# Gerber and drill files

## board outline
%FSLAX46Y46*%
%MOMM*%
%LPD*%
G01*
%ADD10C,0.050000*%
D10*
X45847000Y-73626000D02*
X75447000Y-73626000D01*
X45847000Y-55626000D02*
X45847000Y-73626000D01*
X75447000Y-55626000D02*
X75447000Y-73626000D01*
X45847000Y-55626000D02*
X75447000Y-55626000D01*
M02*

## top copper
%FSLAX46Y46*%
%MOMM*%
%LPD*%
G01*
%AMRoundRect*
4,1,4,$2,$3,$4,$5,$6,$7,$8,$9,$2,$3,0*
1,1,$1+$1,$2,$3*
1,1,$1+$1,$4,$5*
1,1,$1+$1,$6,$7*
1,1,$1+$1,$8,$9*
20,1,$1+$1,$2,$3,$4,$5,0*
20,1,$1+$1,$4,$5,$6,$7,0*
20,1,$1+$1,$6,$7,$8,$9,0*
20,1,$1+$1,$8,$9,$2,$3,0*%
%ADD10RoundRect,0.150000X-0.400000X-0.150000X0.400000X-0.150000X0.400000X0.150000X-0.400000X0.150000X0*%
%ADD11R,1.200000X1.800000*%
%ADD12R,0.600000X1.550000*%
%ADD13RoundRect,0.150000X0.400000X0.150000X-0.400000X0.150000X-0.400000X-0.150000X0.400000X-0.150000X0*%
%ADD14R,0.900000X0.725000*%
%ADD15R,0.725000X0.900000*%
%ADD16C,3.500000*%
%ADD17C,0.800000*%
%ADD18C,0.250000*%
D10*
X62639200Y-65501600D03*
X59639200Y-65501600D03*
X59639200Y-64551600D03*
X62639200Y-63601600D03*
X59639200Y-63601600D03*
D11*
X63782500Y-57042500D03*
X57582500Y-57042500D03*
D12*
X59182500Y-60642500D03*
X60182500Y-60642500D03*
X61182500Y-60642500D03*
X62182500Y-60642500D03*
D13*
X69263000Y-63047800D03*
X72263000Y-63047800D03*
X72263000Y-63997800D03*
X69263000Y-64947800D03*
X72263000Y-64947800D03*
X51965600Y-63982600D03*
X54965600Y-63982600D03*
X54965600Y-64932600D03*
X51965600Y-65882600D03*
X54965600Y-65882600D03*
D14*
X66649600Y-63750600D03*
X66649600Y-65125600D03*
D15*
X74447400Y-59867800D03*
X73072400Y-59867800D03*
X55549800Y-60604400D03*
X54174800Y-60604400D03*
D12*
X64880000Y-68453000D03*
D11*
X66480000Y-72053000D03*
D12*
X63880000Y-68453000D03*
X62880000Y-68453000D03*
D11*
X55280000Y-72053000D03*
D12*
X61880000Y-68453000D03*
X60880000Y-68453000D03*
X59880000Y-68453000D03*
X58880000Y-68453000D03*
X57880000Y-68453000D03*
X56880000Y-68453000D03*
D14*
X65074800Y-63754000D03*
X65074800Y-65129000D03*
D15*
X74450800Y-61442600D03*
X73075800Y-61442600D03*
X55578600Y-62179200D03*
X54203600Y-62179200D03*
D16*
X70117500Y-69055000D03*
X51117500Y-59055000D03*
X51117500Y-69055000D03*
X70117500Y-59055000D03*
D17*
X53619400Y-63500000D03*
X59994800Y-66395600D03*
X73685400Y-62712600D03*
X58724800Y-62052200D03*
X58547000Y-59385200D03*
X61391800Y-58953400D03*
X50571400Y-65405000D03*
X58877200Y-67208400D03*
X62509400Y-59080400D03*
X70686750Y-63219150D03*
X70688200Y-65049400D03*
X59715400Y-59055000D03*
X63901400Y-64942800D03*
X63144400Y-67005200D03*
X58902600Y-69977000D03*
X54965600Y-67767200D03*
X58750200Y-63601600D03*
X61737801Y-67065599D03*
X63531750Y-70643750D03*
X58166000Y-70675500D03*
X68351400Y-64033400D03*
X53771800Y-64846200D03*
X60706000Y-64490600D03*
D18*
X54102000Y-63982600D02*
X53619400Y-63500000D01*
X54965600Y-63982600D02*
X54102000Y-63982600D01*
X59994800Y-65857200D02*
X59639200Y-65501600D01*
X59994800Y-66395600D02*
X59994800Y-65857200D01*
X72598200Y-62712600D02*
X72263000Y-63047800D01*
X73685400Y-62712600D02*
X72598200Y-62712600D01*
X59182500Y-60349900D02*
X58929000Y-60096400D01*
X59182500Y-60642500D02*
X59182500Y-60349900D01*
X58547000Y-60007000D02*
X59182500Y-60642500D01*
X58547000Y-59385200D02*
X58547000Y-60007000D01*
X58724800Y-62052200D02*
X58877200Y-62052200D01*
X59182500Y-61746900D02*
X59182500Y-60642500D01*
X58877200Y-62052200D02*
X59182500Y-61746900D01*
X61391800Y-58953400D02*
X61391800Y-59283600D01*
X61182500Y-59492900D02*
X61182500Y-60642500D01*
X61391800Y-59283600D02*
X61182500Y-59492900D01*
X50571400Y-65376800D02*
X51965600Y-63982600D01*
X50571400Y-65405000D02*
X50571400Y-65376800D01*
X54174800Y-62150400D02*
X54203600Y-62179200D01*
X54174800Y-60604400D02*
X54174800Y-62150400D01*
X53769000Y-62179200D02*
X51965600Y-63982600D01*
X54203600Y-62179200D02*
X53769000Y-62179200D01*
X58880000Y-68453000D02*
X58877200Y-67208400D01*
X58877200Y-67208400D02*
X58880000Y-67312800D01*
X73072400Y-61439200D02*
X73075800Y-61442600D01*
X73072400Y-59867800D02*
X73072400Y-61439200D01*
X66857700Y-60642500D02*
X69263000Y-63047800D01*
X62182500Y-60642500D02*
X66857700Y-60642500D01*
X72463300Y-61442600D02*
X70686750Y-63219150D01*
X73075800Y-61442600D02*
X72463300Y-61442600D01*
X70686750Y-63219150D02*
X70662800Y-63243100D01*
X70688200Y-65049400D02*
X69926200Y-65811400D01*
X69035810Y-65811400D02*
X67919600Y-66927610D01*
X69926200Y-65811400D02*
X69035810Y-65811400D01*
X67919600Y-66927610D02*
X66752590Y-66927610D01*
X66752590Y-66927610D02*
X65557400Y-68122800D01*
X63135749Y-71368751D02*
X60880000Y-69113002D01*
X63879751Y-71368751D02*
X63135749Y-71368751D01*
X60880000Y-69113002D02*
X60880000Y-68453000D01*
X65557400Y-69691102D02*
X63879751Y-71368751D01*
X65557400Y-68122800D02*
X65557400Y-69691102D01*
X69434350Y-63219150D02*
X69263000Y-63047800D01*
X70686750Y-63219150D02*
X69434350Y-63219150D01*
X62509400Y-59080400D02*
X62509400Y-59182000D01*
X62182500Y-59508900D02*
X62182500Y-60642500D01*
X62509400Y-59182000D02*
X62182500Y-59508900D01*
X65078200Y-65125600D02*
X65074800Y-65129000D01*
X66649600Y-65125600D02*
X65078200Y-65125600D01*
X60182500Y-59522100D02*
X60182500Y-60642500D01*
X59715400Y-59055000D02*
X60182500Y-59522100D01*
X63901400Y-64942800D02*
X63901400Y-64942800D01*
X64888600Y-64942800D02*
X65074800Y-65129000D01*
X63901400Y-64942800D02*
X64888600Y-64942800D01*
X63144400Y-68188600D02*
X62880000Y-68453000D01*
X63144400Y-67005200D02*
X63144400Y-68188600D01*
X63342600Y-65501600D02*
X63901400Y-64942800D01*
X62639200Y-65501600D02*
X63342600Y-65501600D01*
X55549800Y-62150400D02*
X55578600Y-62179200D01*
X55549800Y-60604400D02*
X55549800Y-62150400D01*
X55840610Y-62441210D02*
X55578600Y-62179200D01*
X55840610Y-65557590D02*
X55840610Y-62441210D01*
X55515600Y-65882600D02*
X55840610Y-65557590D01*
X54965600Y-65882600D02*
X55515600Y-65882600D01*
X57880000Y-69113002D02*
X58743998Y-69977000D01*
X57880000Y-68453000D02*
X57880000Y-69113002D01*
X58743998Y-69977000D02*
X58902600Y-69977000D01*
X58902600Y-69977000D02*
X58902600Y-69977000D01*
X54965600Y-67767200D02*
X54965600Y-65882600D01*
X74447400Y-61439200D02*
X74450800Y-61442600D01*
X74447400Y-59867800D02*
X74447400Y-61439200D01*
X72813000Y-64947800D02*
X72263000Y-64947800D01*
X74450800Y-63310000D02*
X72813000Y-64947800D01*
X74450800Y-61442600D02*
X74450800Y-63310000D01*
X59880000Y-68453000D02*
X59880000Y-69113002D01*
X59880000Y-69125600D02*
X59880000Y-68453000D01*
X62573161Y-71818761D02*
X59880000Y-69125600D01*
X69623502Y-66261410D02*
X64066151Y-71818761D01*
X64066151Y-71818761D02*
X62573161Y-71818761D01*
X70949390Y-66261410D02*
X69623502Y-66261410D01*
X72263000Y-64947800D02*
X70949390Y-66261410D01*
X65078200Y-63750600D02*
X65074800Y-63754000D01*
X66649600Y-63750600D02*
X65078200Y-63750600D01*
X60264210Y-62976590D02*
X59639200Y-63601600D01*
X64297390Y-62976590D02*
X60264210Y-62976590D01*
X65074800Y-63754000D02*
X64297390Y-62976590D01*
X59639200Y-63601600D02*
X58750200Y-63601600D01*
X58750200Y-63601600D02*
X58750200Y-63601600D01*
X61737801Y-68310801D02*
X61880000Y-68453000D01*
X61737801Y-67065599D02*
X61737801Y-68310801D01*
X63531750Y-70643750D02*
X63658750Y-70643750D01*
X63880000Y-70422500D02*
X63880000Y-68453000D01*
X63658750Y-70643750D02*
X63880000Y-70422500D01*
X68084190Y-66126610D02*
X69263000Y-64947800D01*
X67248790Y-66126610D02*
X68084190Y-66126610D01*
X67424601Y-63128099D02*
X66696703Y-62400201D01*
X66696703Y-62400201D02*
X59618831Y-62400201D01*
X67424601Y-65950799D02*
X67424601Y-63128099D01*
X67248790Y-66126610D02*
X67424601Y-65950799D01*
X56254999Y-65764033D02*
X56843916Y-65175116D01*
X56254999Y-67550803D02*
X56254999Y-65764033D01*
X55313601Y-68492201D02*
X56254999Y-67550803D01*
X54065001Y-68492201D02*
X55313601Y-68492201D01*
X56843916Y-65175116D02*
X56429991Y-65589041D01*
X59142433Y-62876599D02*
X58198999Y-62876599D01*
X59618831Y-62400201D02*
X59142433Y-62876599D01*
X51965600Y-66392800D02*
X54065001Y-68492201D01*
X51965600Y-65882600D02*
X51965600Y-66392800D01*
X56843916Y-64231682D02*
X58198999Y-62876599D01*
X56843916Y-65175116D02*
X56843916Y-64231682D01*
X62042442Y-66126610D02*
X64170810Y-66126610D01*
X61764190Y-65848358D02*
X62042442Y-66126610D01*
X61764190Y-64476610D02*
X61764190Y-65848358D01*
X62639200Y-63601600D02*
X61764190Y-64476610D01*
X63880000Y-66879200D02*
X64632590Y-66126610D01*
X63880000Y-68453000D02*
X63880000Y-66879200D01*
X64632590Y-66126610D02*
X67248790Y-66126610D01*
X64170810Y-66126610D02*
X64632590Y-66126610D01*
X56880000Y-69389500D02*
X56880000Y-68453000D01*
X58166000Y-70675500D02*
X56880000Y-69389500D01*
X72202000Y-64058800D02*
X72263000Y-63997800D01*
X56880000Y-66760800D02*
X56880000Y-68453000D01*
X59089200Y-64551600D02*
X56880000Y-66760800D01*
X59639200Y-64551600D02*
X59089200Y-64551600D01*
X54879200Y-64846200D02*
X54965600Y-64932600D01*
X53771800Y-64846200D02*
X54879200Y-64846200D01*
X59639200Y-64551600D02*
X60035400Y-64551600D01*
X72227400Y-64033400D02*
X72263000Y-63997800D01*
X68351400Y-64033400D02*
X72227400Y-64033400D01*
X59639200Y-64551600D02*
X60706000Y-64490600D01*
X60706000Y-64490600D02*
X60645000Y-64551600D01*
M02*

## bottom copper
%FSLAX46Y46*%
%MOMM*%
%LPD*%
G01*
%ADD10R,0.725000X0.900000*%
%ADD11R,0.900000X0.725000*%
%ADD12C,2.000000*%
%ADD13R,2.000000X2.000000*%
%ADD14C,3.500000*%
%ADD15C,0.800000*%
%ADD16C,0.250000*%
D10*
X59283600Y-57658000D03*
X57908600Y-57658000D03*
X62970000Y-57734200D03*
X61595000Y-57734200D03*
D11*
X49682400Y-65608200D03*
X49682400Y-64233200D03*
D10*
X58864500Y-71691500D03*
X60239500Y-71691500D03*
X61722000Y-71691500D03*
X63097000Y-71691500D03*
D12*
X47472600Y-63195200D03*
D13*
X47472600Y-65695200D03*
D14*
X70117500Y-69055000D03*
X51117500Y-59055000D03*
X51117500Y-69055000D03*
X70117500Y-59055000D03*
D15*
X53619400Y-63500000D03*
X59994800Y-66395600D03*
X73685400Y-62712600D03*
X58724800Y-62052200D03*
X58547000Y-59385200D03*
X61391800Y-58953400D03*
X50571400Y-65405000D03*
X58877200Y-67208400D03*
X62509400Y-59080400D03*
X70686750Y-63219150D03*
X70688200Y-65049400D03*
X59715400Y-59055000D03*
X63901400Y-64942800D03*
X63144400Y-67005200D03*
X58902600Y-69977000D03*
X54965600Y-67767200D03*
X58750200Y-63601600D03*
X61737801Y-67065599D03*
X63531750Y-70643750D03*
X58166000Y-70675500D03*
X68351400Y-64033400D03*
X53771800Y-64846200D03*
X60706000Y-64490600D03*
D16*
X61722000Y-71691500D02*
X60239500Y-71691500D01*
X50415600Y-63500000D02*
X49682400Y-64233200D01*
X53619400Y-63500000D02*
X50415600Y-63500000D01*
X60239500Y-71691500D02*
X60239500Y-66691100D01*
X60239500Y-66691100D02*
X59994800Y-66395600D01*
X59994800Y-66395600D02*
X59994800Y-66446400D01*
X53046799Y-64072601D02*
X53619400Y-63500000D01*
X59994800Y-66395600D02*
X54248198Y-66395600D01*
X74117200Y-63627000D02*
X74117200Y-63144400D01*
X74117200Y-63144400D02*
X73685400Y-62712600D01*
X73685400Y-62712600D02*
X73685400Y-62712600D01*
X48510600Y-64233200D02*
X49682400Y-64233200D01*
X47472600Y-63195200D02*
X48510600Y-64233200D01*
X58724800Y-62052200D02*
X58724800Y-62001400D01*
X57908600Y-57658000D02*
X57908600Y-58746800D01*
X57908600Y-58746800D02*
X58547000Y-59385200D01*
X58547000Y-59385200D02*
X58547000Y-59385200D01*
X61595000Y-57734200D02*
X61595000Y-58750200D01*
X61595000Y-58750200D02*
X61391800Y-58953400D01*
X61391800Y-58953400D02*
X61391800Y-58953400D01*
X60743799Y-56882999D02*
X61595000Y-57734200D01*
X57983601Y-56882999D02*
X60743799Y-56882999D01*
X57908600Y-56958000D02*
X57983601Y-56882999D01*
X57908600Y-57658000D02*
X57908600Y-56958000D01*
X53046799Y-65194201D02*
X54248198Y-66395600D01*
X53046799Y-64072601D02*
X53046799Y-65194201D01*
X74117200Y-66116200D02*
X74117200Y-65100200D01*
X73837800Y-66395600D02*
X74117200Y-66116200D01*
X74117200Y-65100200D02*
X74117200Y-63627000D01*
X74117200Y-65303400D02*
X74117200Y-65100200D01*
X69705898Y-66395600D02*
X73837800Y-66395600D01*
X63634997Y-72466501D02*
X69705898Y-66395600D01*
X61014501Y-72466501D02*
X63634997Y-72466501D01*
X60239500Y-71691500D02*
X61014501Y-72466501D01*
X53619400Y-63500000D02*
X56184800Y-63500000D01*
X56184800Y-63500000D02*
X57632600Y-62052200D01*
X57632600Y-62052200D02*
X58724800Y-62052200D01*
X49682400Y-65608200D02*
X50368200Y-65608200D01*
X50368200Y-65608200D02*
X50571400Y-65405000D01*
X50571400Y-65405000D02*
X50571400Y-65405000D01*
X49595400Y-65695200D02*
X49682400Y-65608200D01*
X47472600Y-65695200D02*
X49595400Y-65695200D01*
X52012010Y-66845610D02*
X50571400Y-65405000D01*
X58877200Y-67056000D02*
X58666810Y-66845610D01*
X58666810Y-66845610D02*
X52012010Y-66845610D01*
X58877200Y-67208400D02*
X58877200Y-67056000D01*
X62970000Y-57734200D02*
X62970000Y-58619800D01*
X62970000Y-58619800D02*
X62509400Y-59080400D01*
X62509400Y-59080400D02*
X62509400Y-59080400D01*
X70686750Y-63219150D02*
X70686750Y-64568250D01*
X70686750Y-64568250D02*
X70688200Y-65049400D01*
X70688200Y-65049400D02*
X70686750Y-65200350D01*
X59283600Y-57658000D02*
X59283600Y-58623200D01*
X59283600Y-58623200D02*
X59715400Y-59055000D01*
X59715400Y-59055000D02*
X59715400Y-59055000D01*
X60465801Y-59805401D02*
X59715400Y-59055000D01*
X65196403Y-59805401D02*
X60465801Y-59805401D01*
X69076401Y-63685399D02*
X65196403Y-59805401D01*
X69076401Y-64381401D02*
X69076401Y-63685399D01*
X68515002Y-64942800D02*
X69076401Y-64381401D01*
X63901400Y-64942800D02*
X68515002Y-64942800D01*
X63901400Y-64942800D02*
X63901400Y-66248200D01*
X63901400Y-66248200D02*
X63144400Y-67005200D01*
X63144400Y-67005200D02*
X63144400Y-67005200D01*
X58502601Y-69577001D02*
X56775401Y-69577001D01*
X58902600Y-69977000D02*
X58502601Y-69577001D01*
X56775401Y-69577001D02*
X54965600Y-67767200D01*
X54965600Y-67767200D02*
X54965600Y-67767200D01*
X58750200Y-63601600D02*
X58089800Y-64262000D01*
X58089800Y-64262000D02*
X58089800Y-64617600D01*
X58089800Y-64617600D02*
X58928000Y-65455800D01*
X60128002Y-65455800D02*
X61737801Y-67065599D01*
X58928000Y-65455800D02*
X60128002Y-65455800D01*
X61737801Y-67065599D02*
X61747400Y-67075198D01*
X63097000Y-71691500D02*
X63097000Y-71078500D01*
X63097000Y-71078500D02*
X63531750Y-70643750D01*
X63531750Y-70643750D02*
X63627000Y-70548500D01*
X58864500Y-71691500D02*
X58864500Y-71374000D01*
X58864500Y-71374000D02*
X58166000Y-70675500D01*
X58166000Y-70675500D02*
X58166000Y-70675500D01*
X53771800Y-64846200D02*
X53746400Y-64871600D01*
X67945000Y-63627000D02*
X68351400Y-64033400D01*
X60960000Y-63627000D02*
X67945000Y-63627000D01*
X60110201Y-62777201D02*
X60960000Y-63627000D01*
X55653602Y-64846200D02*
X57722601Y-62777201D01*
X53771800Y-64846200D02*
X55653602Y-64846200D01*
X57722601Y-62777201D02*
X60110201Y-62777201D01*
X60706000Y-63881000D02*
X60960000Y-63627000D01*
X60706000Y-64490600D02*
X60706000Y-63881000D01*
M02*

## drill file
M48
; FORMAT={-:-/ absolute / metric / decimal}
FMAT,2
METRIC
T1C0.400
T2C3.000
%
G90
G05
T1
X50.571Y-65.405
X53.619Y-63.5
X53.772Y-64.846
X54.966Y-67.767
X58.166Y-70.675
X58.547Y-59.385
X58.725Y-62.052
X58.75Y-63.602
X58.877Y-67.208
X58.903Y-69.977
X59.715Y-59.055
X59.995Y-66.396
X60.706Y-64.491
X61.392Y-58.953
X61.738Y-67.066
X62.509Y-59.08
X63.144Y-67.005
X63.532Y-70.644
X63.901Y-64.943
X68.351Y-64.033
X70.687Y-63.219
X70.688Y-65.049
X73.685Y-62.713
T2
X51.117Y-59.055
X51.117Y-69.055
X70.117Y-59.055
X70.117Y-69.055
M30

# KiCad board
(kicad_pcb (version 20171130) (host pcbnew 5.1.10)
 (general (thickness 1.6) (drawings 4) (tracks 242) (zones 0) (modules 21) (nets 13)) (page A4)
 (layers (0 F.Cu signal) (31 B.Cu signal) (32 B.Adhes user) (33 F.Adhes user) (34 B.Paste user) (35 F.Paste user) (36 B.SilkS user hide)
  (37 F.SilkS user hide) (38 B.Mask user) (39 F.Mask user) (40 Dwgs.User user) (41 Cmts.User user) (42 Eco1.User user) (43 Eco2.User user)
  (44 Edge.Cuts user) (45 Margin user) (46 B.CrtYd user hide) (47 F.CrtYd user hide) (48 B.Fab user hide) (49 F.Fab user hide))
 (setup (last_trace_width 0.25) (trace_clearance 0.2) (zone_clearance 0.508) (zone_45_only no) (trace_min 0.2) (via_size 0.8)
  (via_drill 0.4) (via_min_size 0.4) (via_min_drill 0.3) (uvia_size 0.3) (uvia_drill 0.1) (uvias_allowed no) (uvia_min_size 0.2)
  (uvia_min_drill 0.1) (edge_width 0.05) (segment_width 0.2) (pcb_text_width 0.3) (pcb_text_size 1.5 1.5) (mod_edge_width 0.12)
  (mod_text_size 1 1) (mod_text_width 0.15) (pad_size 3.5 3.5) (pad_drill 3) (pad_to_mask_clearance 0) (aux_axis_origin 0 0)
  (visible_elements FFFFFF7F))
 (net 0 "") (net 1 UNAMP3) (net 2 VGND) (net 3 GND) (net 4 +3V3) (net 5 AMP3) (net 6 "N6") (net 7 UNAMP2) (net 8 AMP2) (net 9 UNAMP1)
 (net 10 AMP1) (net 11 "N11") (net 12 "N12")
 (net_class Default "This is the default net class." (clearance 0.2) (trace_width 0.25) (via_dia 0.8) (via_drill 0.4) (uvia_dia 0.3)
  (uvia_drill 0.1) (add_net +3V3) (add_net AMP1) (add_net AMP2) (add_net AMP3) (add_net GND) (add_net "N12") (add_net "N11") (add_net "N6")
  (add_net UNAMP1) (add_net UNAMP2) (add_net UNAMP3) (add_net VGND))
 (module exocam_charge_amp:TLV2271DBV (layer F.Cu) (at 60.9092 61.0616)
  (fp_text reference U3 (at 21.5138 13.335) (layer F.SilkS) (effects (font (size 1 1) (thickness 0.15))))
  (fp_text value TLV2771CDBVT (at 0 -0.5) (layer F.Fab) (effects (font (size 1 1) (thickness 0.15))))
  (pad 4 smd roundrect (at 1.73 4.44) (size 1.1 0.6) (layers F.Cu F.Paste F.Mask) (roundrect_rratio 0.25) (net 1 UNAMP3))
  (pad 3 smd roundrect (at -1.27 4.44) (size 1.1 0.6) (layers F.Cu F.Paste F.Mask) (roundrect_rratio 0.25) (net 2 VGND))
  (pad 2 smd roundrect (at -1.27 3.49) (size 1.1 0.6) (layers F.Cu F.Paste F.Mask) (roundrect_rratio 0.25) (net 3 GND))
  (pad 5 smd roundrect (at 1.73 2.54) (size 1.1 0.6) (layers F.Cu F.Paste F.Mask) (roundrect_rratio 0.25) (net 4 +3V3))
  (pad 1 smd roundrect (at -1.27 2.54) (size 1.1 0.6) (layers F.Cu F.Paste F.Mask) (roundrect_rratio 0.25) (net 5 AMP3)))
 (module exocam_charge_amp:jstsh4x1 (layer F.Cu) (at 59.3725 63.1825 180)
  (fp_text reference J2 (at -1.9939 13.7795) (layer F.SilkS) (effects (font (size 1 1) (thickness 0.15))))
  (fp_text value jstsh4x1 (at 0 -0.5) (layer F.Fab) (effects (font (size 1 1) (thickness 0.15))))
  (pad 5 smd rect (at -4.41 6.14 180) (size 1.2 1.8) (layers F.Cu F.Paste F.Mask) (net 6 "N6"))
  (pad 5 smd rect (at 1.79 6.14 180) (size 1.2 1.8) (layers F.Cu F.Paste F.Mask) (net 6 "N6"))
  (pad 4 smd rect (at 0.19 2.54 180) (size 0.6 1.55) (layers F.Cu F.Paste F.Mask) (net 2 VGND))
  (pad 3 smd rect (at -0.81 2.54 180) (size 0.6 1.55) (layers F.Cu F.Paste F.Mask) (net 1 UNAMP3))
  (pad 2 smd rect (at -1.81 2.54 180) (size 0.6 1.55) (layers F.Cu F.Paste F.Mask) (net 2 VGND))
  (pad 1 smd rect (at -2.81 2.54 180) (size 0.6 1.55) (layers F.Cu F.Paste F.Mask) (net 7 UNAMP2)))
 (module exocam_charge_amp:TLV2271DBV (layer F.Cu) (at 70.993 67.4878 180)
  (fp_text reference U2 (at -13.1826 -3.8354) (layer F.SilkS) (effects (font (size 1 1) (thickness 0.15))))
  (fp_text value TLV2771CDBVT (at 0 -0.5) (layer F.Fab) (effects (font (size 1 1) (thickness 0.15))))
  (pad 4 smd roundrect (at 1.73 4.44 180) (size 1.1 0.6) (layers F.Cu F.Paste F.Mask) (roundrect_rratio 0.25) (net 7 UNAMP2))
  (pad 3 smd roundrect (at -1.27 4.44 180) (size 1.1 0.6) (layers F.Cu F.Paste F.Mask) (roundrect_rratio 0.25) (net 2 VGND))
  (pad 2 smd roundrect (at -1.27 3.49 180) (size 1.1 0.6) (layers F.Cu F.Paste F.Mask) (roundrect_rratio 0.25) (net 3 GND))
  (pad 5 smd roundrect (at 1.73 2.54 180) (size 1.1 0.6) (layers F.Cu F.Paste F.Mask) (roundrect_rratio 0.25) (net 4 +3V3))
  (pad 1 smd roundrect (at -1.27 2.54 180) (size 1.1 0.6) (layers F.Cu F.Paste F.Mask) (roundrect_rratio 0.25) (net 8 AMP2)))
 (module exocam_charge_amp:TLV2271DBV (layer F.Cu) (at 53.6956 68.4226 180)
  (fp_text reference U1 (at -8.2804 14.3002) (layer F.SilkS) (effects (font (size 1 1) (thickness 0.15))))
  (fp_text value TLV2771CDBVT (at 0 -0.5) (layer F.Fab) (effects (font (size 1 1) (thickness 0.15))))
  (pad 4 smd roundrect (at 1.73 4.44 180) (size 1.1 0.6) (layers F.Cu F.Paste F.Mask) (roundrect_rratio 0.25) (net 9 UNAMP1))
  (pad 3 smd roundrect (at -1.27 4.44 180) (size 1.1 0.6) (layers F.Cu F.Paste F.Mask) (roundrect_rratio 0.25) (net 2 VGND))
  (pad 2 smd roundrect (at -1.27 3.49 180) (size 1.1 0.6) (layers F.Cu F.Paste F.Mask) (roundrect_rratio 0.25) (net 3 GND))
  (pad 5 smd roundrect (at 1.73 2.54 180) (size 1.1 0.6) (layers F.Cu F.Paste F.Mask) (roundrect_rratio 0.25) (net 4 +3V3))
  (pad 1 smd roundrect (at -1.27 2.54 180) (size 1.1 0.6) (layers F.Cu F.Paste F.Mask) (roundrect_rratio 0.25) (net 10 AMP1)))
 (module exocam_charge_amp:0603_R (layer F.Cu) (at 64.1096 63.8556 90)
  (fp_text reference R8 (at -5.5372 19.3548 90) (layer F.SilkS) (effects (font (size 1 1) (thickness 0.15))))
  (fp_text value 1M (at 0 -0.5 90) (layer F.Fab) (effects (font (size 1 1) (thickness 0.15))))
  (pad 2 smd rect (at 0.105 2.54 90) (size 0.725 0.9) (layers F.Cu F.Paste F.Mask) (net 5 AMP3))
  (pad 1 smd rect (at -1.27 2.54 90) (size 0.725 0.9) (layers F.Cu F.Paste F.Mask) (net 1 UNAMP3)))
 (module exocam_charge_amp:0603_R (layer B.Cu) (at 59.1786 60.198)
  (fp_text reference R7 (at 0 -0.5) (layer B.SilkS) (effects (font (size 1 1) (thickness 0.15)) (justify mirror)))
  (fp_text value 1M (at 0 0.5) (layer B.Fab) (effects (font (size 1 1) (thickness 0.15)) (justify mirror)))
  (pad 2 smd rect (at 0.105 -2.54) (size 0.725 0.9) (layers B.Cu B.Paste B.Mask) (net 1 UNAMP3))
  (pad 1 smd rect (at -1.27 -2.54) (size 0.725 0.9) (layers B.Cu B.Paste B.Mask) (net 2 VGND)))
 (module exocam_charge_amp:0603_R (layer F.Cu) (at 74.3424 57.3278)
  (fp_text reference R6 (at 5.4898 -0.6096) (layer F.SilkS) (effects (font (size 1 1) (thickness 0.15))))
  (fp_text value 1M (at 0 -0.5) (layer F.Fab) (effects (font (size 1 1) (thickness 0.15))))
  (pad 2 smd rect (at 0.105 2.54) (size 0.725 0.9) (layers F.Cu F.Paste F.Mask) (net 8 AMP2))
  (pad 1 smd rect (at -1.27 2.54) (size 0.725 0.9) (layers F.Cu F.Paste F.Mask) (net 7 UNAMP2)))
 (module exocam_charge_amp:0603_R (layer B.Cu) (at 62.865 60.2742)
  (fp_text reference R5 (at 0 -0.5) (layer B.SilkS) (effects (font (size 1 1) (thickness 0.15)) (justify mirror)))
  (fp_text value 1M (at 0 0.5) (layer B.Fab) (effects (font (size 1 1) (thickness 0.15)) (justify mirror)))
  (pad 2 smd rect (at 0.105 -2.54) (size 0.725 0.9) (layers B.Cu B.Paste B.Mask) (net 7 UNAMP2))
  (pad 1 smd rect (at -1.27 -2.54) (size 0.725 0.9) (layers B.Cu B.Paste B.Mask) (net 2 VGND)))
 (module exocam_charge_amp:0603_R (layer B.Cu) (at 47.1424 65.5032 270)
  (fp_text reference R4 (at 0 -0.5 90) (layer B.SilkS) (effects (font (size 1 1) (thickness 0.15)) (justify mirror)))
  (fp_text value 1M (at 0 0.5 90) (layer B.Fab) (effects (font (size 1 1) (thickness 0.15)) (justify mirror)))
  (pad 2 smd rect (at 0.105 -2.54 270) (size 0.725 0.9) (layers B.Cu B.Paste B.Mask) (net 9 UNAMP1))
  (pad 1 smd rect (at -1.27 -2.54 270) (size 0.725 0.9) (layers B.Cu B.Paste B.Mask) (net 2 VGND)))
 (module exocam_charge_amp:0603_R (layer F.Cu) (at 55.4448 58.0644)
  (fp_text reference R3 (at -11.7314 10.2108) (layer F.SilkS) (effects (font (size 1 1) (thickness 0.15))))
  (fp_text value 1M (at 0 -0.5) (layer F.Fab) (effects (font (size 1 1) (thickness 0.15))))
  (pad 2 smd rect (at 0.105 2.54) (size 0.725 0.9) (layers F.Cu F.Paste F.Mask) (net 10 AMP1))
  (pad 1 smd rect (at -1.27 2.54) (size 0.725 0.9) (layers F.Cu F.Paste F.Mask) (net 9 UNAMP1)))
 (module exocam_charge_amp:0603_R (layer B.Cu) (at 58.9695 69.1515 180)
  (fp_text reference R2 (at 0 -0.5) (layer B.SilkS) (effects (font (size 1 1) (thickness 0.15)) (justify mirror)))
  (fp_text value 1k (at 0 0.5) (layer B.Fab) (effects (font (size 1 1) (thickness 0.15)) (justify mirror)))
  (pad 2 smd rect (at 0.105 -2.54 180) (size 0.725 0.9) (layers B.Cu B.Paste B.Mask) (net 3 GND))
  (pad 1 smd rect (at -1.27 -2.54 180) (size 0.725 0.9) (layers B.Cu B.Paste B.Mask) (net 2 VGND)))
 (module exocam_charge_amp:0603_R (layer B.Cu) (at 61.827 69.1515 180)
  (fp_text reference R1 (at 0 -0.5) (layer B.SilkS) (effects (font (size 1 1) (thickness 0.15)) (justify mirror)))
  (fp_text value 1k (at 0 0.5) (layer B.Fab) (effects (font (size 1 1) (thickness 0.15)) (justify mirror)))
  (pad 2 smd rect (at 0.105 -2.54 180) (size 0.725 0.9) (layers B.Cu B.Paste B.Mask) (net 2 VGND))
  (pad 1 smd rect (at -1.27 -2.54 180) (size 0.725 0.9) (layers B.Cu B.Paste B.Mask) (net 4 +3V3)))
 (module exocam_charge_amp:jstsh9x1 (layer F.Cu) (at 59.69 65.913)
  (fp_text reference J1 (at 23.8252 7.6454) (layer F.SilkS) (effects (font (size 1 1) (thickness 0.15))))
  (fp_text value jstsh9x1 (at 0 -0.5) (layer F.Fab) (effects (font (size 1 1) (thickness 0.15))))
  (pad 9 smd rect (at 5.19 2.54) (size 0.6 1.55) (layers F.Cu F.Paste F.Mask) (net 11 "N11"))
  (pad 10 smd rect (at 6.79 6.14) (size 1.2 1.8) (layers F.Cu F.Paste F.Mask) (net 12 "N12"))
  (pad 8 smd rect (at 4.19 2.54) (size 0.6 1.55) (layers F.Cu F.Paste F.Mask) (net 4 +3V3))
  (pad 7 smd rect (at 3.19 2.54) (size 0.6 1.55) (layers F.Cu F.Paste F.Mask) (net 1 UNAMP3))
  (pad 10 smd rect (at -4.41 6.14) (size 1.2 1.8) (layers F.Cu F.Paste F.Mask) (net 12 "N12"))
  (pad 6 smd rect (at 2.19 2.54) (size 0.6 1.55) (layers F.Cu F.Paste F.Mask) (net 5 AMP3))
  (pad 5 smd rect (at 1.19 2.54) (size 0.6 1.55) (layers F.Cu F.Paste F.Mask) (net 7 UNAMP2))
  (pad 4 smd rect (at 0.19 2.54) (size 0.6 1.55) (layers F.Cu F.Paste F.Mask) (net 8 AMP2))
  (pad 3 smd rect (at -0.81 2.54) (size 0.6 1.55) (layers F.Cu F.Paste F.Mask) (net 9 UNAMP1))
  (pad 2 smd rect (at -1.81 2.54) (size 0.6 1.55) (layers F.Cu F.Paste F.Mask) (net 10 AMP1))
  (pad 1 smd rect (at -2.81 2.54) (size 0.6 1.55) (layers F.Cu F.Paste F.Mask) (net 3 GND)))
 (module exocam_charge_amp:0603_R (layer F.Cu) (at 62.5348 63.859 90)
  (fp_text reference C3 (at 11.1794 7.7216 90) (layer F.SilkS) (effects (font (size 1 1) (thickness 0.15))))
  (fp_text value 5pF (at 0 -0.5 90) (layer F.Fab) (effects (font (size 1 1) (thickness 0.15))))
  (pad 2 smd rect (at 0.105 2.54 90) (size 0.725 0.9) (layers F.Cu F.Paste F.Mask) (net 5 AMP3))
  (pad 1 smd rect (at -1.27 2.54 90) (size 0.725 0.9) (layers F.Cu F.Paste F.Mask) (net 1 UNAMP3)))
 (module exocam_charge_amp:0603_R (layer F.Cu) (at 74.3458 58.9026)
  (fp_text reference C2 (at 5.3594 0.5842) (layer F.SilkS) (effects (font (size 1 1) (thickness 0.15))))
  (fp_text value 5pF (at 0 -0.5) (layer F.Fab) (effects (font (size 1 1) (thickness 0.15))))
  (pad 2 smd rect (at 0.105 2.54) (size 0.725 0.9) (layers F.Cu F.Paste F.Mask) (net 8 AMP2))
  (pad 1 smd rect (at -1.27 2.54) (size 0.725 0.9) (layers F.Cu F.Paste F.Mask) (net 7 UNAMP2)))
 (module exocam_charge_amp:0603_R (layer F.Cu) (at 55.4736 59.6392)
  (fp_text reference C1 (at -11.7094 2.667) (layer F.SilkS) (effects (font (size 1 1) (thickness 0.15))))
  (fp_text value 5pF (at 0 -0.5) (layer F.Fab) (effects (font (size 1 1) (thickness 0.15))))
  (pad 2 smd rect (at 0.105 2.54) (size 0.725 0.9) (layers F.Cu F.Paste F.Mask) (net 10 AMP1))
  (pad 1 smd rect (at -1.27 2.54) (size 0.725 0.9) (layers F.Cu F.Paste F.Mask) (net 9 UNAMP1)))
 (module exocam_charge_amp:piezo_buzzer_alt (layer B.Cu) (at 50.0126 64.1552 90)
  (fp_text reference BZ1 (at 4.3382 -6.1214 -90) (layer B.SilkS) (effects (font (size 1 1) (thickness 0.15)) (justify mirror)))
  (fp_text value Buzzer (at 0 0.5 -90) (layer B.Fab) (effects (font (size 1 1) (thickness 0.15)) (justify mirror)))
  (pad 2 smd circle (at 0.96 -2.54 90) (size 2 2) (layers B.Cu B.Paste B.Mask) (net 2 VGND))
  (pad 1 smd rect (at -1.54 -2.54 90) (size 2 2) (layers B.Cu B.Paste B.Mask) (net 9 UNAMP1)))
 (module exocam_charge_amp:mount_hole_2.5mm (layer F.Cu) (at 66.1035 71.501 90)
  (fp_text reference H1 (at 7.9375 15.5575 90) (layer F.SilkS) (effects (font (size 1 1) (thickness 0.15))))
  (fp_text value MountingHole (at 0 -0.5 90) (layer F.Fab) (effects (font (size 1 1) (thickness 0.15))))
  (pad 1 thru_hole circle (at 2.446 4.014 90) (size 3.5 3.5) (drill 3) (layers *.Cu *.Mask)))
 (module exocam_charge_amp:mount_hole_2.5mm (layer F.Cu) (at 47.3075 57.785 90)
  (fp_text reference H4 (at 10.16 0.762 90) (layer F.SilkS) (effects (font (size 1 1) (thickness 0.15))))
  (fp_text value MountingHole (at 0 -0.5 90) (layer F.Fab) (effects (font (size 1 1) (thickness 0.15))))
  (pad 1 thru_hole circle (at -1.27 3.81 90) (size 3.5 3.5) (drill 3) (layers *.Cu *.Mask)))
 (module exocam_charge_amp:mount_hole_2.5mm (layer F.Cu) (at 47.3075 60.96 90)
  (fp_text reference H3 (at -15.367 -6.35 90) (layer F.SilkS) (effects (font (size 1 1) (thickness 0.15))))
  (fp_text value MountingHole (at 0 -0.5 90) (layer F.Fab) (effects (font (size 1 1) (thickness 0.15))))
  (pad 1 thru_hole circle (at -8.095 3.81 90) (size 3.5 3.5) (drill 3) (layers *.Cu *.Mask)))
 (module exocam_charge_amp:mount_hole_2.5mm (layer F.Cu) (at 66.1035 57.501 90)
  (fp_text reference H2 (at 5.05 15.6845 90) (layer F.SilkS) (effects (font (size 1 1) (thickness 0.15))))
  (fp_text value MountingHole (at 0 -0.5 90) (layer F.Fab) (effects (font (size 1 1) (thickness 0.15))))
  (pad 1 thru_hole circle (at -1.554 4.014 90) (size 3.5 3.5) (drill 3) (layers *.Cu *.Mask)))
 (gr_line (start 45.847 73.626) (end 75.447 73.626) (layer Edge.Cuts) (width 0.05))
 (gr_line (start 45.847 55.626) (end 45.847 73.626) (layer Edge.Cuts) (width 0.05))
 (gr_line (start 75.447 55.626) (end 75.447 73.626) (layer Edge.Cuts) (width 0.05))
 (gr_line (start 45.847 55.626) (end 75.447 55.626) (layer Edge.Cuts) (width 0.05))
 (segment (start 61.722 71.6915) (end 60.2395 71.6915) (width 0.25) (layer B.Cu) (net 2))
 (via (at 53.6194 63.5) (size 0.8) (drill 0.4) (layers F.Cu B.Cu) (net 2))
 (segment (start 54.102 63.9826) (end 53.6194 63.5) (width 0.25) (layer F.Cu) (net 2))
 (segment (start 54.9656 63.9826) (end 54.102 63.9826) (width 0.25) (layer F.Cu) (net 2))
 (segment (start 50.4156 63.5) (end 49.6824 64.2332) (width 0.25) (layer B.Cu) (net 2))
 (segment (start 53.6194 63.5) (end 50.4156 63.5) (width 0.25) (layer B.Cu) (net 2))
 (segment (start 60.2395 71.6915) (end 60.2395 66.6911) (width 0.25) (layer B.Cu) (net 2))
 (segment (start 60.2395 66.6911) (end 59.9948 66.3956) (width 0.25) (layer B.Cu) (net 2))
 (segment (start 59.9948 66.3956) (end 59.9948 66.4464) (width 0.25) (layer B.Cu) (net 2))
 (via (at 59.9948 66.3956) (size 0.8) (drill 0.4) (layers F.Cu B.Cu) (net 2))
 (segment (start 59.9948 65.8572) (end 59.6392 65.5016) (width 0.25) (layer F.Cu) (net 2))
 (segment (start 59.9948 66.3956) (end 59.9948 65.8572) (width 0.25) (layer F.Cu) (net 2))
 (segment (start 53.046799 64.072601) (end 53.6194 63.5) (width 0.25) (layer B.Cu) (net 2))
 (segment (start 59.9948 66.3956) (end 54.248198 66.3956) (width 0.25) (layer B.Cu) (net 2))
 (segment (start 74.1172 63.627) (end 74.1172 63.1444) (width 0.25) (layer B.Cu) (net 2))
 (segment (start 74.1172 63.1444) (end 73.6854 62.7126) (width 0.25) (layer B.Cu) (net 2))
 (segment (start 73.6854 62.7126) (end 73.6854 62.7126) (width 0.25) (layer B.Cu) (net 2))
 (via (at 73.6854 62.7126) (size 0.8) (drill 0.4) (layers F.Cu B.Cu) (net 2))
 (segment (start 72.5982 62.7126) (end 72.263 63.0478) (width 0.25) (layer F.Cu) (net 2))
 (segment (start 73.6854 62.7126) (end 72.5982 62.7126) (width 0.25) (layer F.Cu) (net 2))
 (segment (start 48.5106 64.2332) (end 49.6824 64.2332) (width 0.25) (layer B.Cu) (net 2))
 (segment (start 47.4726 63.1952) (end 48.5106 64.2332) (width 0.25) (layer B.Cu) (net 2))
 (segment (start 58.7248 62.0522) (end 58.7248 62.0014) (width 0.25) (layer B.Cu) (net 2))
 (via (at 58.7248 62.0522) (size 0.8) (drill 0.4) (layers F.Cu B.Cu) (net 2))
 (segment (start 59.1825 60.3499) (end 58.929 60.0964) (width 0.25) (layer F.Cu) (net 2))
 (segment (start 59.1825 60.6425) (end 59.1825 60.3499) (width 0.25) (layer F.Cu) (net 2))
 (segment (start 57.9086 57.658) (end 57.9086 58.7468) (width 0.25) (layer B.Cu) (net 2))
 (segment (start 57.9086 58.7468) (end 58.547 59.3852) (width 0.25) (layer B.Cu) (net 2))
 (segment (start 58.547 59.3852) (end 58.547 59.3852) (width 0.25) (layer B.Cu) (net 2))
 (via (at 58.547 59.3852) (size 0.8) (drill 0.4) (layers F.Cu B.Cu) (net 2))
 (segment (start 58.547 60.007) (end 59.1825 60.6425) (width 0.25) (layer F.Cu) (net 2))
 (segment (start 58.547 59.3852) (end 58.547 60.007) (width 0.25) (layer F.Cu) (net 2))
 (segment (start 61.595 57.7342) (end 61.595 58.7502) (width 0.25) (layer B.Cu) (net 2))
 (segment (start 61.595 58.7502) (end 61.3918 58.9534) (width 0.25) (layer B.Cu) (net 2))
 (segment (start 61.3918 58.9534) (end 61.3918 58.9534) (width 0.25) (layer B.Cu) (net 2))
 (via (at 61.3918 58.9534) (size 0.8) (drill 0.4) (layers F.Cu B.Cu) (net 2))
 (segment (start 60.743799 56.882999) (end 61.595 57.7342) (width 0.25) (layer B.Cu) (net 2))
 (segment (start 57.983601 56.882999) (end 60.743799 56.882999) (width 0.25) (layer B.Cu) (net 2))
 (segment (start 57.9086 56.958) (end 57.983601 56.882999) (width 0.25) (layer B.Cu) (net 2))
 (segment (start 57.9086 57.658) (end 57.9086 56.958) (width 0.25) (layer B.Cu) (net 2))
 (segment (start 53.046799 65.194201) (end 54.248198 66.3956) (width 0.25) (layer B.Cu) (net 2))
 (segment (start 53.046799 64.072601) (end 53.046799 65.194201) (width 0.25) (layer B.Cu) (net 2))
 (segment (start 74.1172 66.1162) (end 74.1172 65.1002) (width 0.25) (layer B.Cu) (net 2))
 (segment (start 73.8378 66.3956) (end 74.1172 66.1162) (width 0.25) (layer B.Cu) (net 2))
 (segment (start 74.1172 65.1002) (end 74.1172 63.627) (width 0.25) (layer B.Cu) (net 2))
 (segment (start 74.1172 65.3034) (end 74.1172 65.1002) (width 0.25) (layer B.Cu) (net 2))
 (segment (start 69.705898 66.3956) (end 73.8378 66.3956) (width 0.25) (layer B.Cu) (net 2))
 (segment (start 63.634997 72.466501) (end 69.705898 66.3956) (width 0.25) (layer B.Cu) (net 2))
 (segment (start 61.014501 72.466501) (end 63.634997 72.466501) (width 0.25) (layer B.Cu) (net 2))
 (segment (start 60.2395 71.6915) (end 61.014501 72.466501) (width 0.25) (layer B.Cu) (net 2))
 (segment (start 53.6194 63.5) (end 56.1848 63.5) (width 0.25) (layer B.Cu) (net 2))
 (segment (start 56.1848 63.5) (end 57.6326 62.0522) (width 0.25) (layer B.Cu) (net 2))
 (segment (start 57.6326 62.0522) (end 58.7248 62.0522) (width 0.25) (layer B.Cu) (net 2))
 (segment (start 58.7248 62.0522) (end 58.8772 62.0522) (width 0.25) (layer F.Cu) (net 2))
 (segment (start 59.1825 61.7469) (end 59.1825 60.6425) (width 0.25) (layer F.Cu) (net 2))
 (segment (start 58.8772 62.0522) (end 59.1825 61.7469) (width 0.25) (layer F.Cu) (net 2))
 (segment (start 61.3918 58.9534) (end 61.3918 59.2836) (width 0.25) (layer F.Cu) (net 2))
 (segment (start 61.1825 59.4929) (end 61.1825 60.6425) (width 0.25) (layer F.Cu) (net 2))
 (segment (start 61.3918 59.2836) (end 61.1825 59.4929) (width 0.25) (layer F.Cu) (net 2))
 (segment (start 49.6824 65.6082) (end 50.3682 65.6082) (width 0.25) (layer B.Cu) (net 9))
 (segment (start 50.3682 65.6082) (end 50.5714 65.405) (width 0.25) (layer B.Cu) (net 9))
 (segment (start 50.5714 65.405) (end 50.5714 65.405) (width 0.25) (layer B.Cu) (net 9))
 (via (at 50.5714 65.405) (size 0.8) (drill 0.4) (layers F.Cu B.Cu) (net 9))
 (segment (start 50.5714 65.3768) (end 51.9656 63.9826) (width 0.25) (layer F.Cu) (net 9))
 (segment (start 50.5714 65.405) (end 50.5714 65.3768) (width 0.25) (layer F.Cu) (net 9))
 (segment (start 54.1748 62.1504) (end 54.2036 62.1792) (width 0.25) (layer F.Cu) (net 9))
 (segment (start 54.1748 60.6044) (end 54.1748 62.1504) (width 0.25) (layer F.Cu) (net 9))
 (segment (start 53.769 62.1792) (end 51.9656 63.9826) (width 0.25) (layer F.Cu) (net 9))
 (segment (start 54.2036 62.1792) (end 53.769 62.1792) (width 0.25) (layer F.Cu) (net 9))
 (segment (start 49.5954 65.6952) (end 49.6824 65.6082) (width 0.25) (layer B.Cu) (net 9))
 (segment (start 47.4726 65.6952) (end 49.5954 65.6952) (width 0.25) (layer B.Cu) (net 9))
 (segment (start 58.88 68.453) (end 58.8772 67.2084) (width 0.25) (layer F.Cu) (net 9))
 (segment (start 58.8772 67.2084) (end 58.88 67.3128) (width 0.25) (layer F.Cu) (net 9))
 (via (at 58.8772 67.2084) (size 0.8) (drill 0.4) (layers F.Cu B.Cu) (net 9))
 (segment (start 52.01201 66.84561) (end 50.5714 65.405) (width 0.25) (layer B.Cu) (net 9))
 (segment (start 58.8772 67.056) (end 58.66681 66.84561) (width 0.25) (layer B.Cu) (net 9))
 (segment (start 58.66681 66.84561) (end 52.01201 66.84561) (width 0.25) (layer B.Cu) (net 9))
 (segment (start 58.8772 67.2084) (end 58.8772 67.056) (width 0.25) (layer B.Cu) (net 9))
 (segment (start 73.0724 61.4392) (end 73.0758 61.4426) (width 0.25) (layer F.Cu) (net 7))
 (segment (start 73.0724 59.8678) (end 73.0724 61.4392) (width 0.25) (layer F.Cu) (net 7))
 (segment (start 66.8577 60.6425) (end 69.263 63.0478) (width 0.25) (layer F.Cu) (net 7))
 (segment (start 62.1825 60.6425) (end 66.8577 60.6425) (width 0.25) (layer F.Cu) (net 7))
 (segment (start 62.97 57.7342) (end 62.97 58.6198) (width 0.25) (layer B.Cu) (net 7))
 (segment (start 62.97 58.6198) (end 62.5094 59.0804) (width 0.25) (layer B.Cu) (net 7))
 (segment (start 62.5094 59.0804) (end 62.5094 59.0804) (width 0.25) (layer B.Cu) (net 7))
 (via (at 62.5094 59.0804) (size 0.8) (drill 0.4) (layers F.Cu B.Cu) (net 7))
 (segment (start 72.4633 61.4426) (end 70.68675 63.21915) (width 0.25) (layer F.Cu) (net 7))
 (segment (start 73.0758 61.4426) (end 72.4633 61.4426) (width 0.25) (layer F.Cu) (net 7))
 (segment (start 70.68675 63.21915) (end 70.6628 63.2431) (width 0.25) (layer F.Cu) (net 7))
 (via (at 70.68675 63.21915) (size 0.8) (drill 0.4) (layers F.Cu B.Cu) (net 7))
 (segment (start 70.68675 63.21915) (end 70.68675 64.56825) (width 0.25) (layer B.Cu) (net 7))
 (segment (start 70.68675 64.56825) (end 70.6882 65.0494) (width 0.25) (layer B.Cu) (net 7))
 (segment (start 70.6882 65.0494) (end 70.68675 65.20035) (width 0.25) (layer B.Cu) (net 7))
 (via (at 70.6882 65.0494) (size 0.8) (drill 0.4) (layers F.Cu B.Cu) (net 7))
 (segment (start 70.6882 65.0494) (end 69.9262 65.8114) (width 0.25) (layer F.Cu) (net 7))
 (segment (start 69.03581 65.8114) (end 67.9196 66.92761) (width 0.25) (layer F.Cu) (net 7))
 (segment (start 69.9262 65.8114) (end 69.03581 65.8114) (width 0.25) (layer F.Cu) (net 7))
 (segment (start 67.9196 66.92761) (end 66.75259 66.92761) (width 0.25) (layer F.Cu) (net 7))
 (segment (start 66.75259 66.92761) (end 65.5574 68.1228) (width 0.25) (layer F.Cu) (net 7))
 (segment (start 63.135749 71.368751) (end 60.88 69.113002) (width 0.25) (layer F.Cu) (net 7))
 (segment (start 63.879751 71.368751) (end 63.135749 71.368751) (width 0.25) (layer F.Cu) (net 7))
 (segment (start 60.88 69.113002) (end 60.88 68.453) (width 0.25) (layer F.Cu) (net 7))
 (segment (start 65.5574 69.691102) (end 63.879751 71.368751) (width 0.25) (layer F.Cu) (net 7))
 (segment (start 65.5574 68.1228) (end 65.5574 69.691102) (width 0.25) (layer F.Cu) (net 7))
 (segment (start 69.43435 63.21915) (end 69.263 63.0478) (width 0.25) (layer F.Cu) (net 7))
 (segment (start 70.68675 63.21915) (end 69.43435 63.21915) (width 0.25) (layer F.Cu) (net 7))
 (segment (start 62.5094 59.0804) (end 62.5094 59.182) (width 0.25) (layer F.Cu) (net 7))
 (segment (start 62.1825 59.5089) (end 62.1825 60.6425) (width 0.25) (layer F.Cu) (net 7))
 (segment (start 62.5094 59.182) (end 62.1825 59.5089) (width 0.25) (layer F.Cu) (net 7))
 (segment (start 65.0782 65.1256) (end 65.0748 65.129) (width 0.25) (layer F.Cu) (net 1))
 (segment (start 66.6496 65.1256) (end 65.0782 65.1256) (width 0.25) (layer F.Cu) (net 1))
 (segment (start 59.2836 57.658) (end 59.2836 58.6232) (width 0.25) (layer B.Cu) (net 1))
 (segment (start 59.2836 58.6232) (end 59.7154 59.055) (width 0.25) (layer B.Cu) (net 1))
 (segment (start 59.7154 59.055) (end 59.7154 59.055) (width 0.25) (layer B.Cu) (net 1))
 (via (at 59.7154 59.055) (size 0.8) (drill 0.4) (layers F.Cu B.Cu) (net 1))
 (segment (start 60.1825 59.5221) (end 60.1825 60.6425) (width 0.25) (layer F.Cu) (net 1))
 (segment (start 59.7154 59.055) (end 60.1825 59.5221) (width 0.25) (layer F.Cu) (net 1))
 (segment (start 63.9014 64.9428) (end 63.9014 64.9428) (width 0.25) (layer F.Cu) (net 1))
 (via (at 63.9014 64.9428) (size 0.8) (drill 0.4) (layers F.Cu B.Cu) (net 1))
 (segment (start 60.465801 59.805401) (end 59.7154 59.055) (width 0.25) (layer B.Cu) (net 1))
 (segment (start 65.196403 59.805401) (end 60.465801 59.805401) (width 0.25) (layer B.Cu) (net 1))
 (segment (start 69.076401 63.685399) (end 65.196403 59.805401) (width 0.25) (layer B.Cu) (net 1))
 (segment (start 69.076401 64.381401) (end 69.076401 63.685399) (width 0.25) (layer B.Cu) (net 1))
 (segment (start 68.515002 64.9428) (end 69.076401 64.381401) (width 0.25) (layer B.Cu) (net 1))
 (segment (start 63.9014 64.9428) (end 68.515002 64.9428) (width 0.25) (layer B.Cu) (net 1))
 (segment (start 64.8886 64.9428) (end 65.0748 65.129) (width 0.25) (layer F.Cu) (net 1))
 (segment (start 63.9014 64.9428) (end 64.8886 64.9428) (width 0.25) (layer F.Cu) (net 1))
 (segment (start 63.9014 64.9428) (end 63.9014 66.2482) (width 0.25) (layer B.Cu) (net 1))
 (segment (start 63.9014 66.2482) (end 63.1444 67.0052) (width 0.25) (layer B.Cu) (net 1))
 (segment (start 63.1444 67.0052) (end 63.1444 67.0052) (width 0.25) (layer B.Cu) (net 1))
 (via (at 63.1444 67.0052) (size 0.8) (drill 0.4) (layers F.Cu B.Cu) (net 1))
 (segment (start 63.1444 68.1886) (end 62.88 68.453) (width 0.25) (layer F.Cu) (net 1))
 (segment (start 63.1444 67.0052) (end 63.1444 68.1886) (width 0.25) (layer F.Cu) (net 1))
 (segment (start 63.3426 65.5016) (end 63.9014 64.9428) (width 0.25) (layer F.Cu) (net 1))
 (segment (start 62.6392 65.5016) (end 63.3426 65.5016) (width 0.25) (layer F.Cu) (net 1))
 (segment (start 55.5498 62.1504) (end 55.5786 62.1792) (width 0.25) (layer F.Cu) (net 10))
 (segment (start 55.5498 60.6044) (end 55.5498 62.1504) (width 0.25) (layer F.Cu) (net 10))
 (segment (start 55.84061 62.44121) (end 55.5786 62.1792) (width 0.25) (layer F.Cu) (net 10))
 (segment (start 55.84061 65.55759) (end 55.84061 62.44121) (width 0.25) (layer F.Cu) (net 10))
 (segment (start 55.5156 65.8826) (end 55.84061 65.55759) (width 0.25) (layer F.Cu) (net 10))
 (segment (start 54.9656 65.8826) (end 55.5156 65.8826) (width 0.25) (layer F.Cu) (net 10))
 (segment (start 57.88 69.113002) (end 58.743998 69.977) (width 0.25) (layer F.Cu) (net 10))
 (segment (start 57.88 68.453) (end 57.88 69.113002) (width 0.25) (layer F.Cu) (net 10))
 (segment (start 58.743998 69.977) (end 58.9026 69.977) (width 0.25) (layer F.Cu) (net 10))
 (segment (start 58.9026 69.977) (end 58.9026 69.977) (width 0.25) (layer F.Cu) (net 10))
 (via (at 58.9026 69.977) (size 0.8) (drill 0.4) (layers F.Cu B.Cu) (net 10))
 (segment (start 58.502601 69.577001) (end 56.775401 69.577001) (width 0.25) (layer B.Cu) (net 10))
 (segment (start 58.9026 69.977) (end 58.502601 69.577001) (width 0.25) (layer B.Cu) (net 10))
 (segment (start 56.775401 69.577001) (end 54.9656 67.7672) (width 0.25) (layer B.Cu) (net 10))
 (segment (start 54.9656 67.7672) (end 54.9656 67.7672) (width 0.25) (layer B.Cu) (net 10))
 (via (at 54.9656 67.7672) (size 0.8) (drill 0.4) (layers F.Cu B.Cu) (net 10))
 (segment (start 54.9656 67.7672) (end 54.9656 65.8826) (width 0.25) (layer F.Cu) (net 10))
 (segment (start 74.4474 61.4392) (end 74.4508 61.4426) (width 0.25) (layer F.Cu) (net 8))
 (segment (start 74.4474 59.8678) (end 74.4474 61.4392) (width 0.25) (layer F.Cu) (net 8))
 (segment (start 72.813 64.9478) (end 72.263 64.9478) (width 0.25) (layer F.Cu) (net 8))
 (segment (start 74.4508 63.31) (end 72.813 64.9478) (width 0.25) (layer F.Cu) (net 8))
 (segment (start 74.4508 61.4426) (end 74.4508 63.31) (width 0.25) (layer F.Cu) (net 8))
 (segment (start 59.88 68.453) (end 59.88 69.113002) (width 0.25) (layer F.Cu) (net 8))
 (segment (start 59.88 69.1256) (end 59.88 68.453) (width 0.25) (layer F.Cu) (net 8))
 (segment (start 62.573161 71.818761) (end 59.88 69.1256) (width 0.25) (layer F.Cu) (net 8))
 (segment (start 69.623502 66.26141) (end 64.066151 71.818761) (width 0.25) (layer F.Cu) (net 8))
 (segment (start 64.066151 71.818761) (end 62.573161 71.818761) (width 0.25) (layer F.Cu) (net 8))
 (segment (start 70.94939 66.26141) (end 69.623502 66.26141) (width 0.25) (layer F.Cu) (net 8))
 (segment (start 72.263 64.9478) (end 70.94939 66.26141) (width 0.25) (layer F.Cu) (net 8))
 (segment (start 65.0782 63.7506) (end 65.0748 63.754) (width 0.25) (layer F.Cu) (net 5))
 (segment (start 66.6496 63.7506) (end 65.0782 63.7506) (width 0.25) (layer F.Cu) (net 5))
 (segment (start 60.26421 62.97659) (end 59.6392 63.6016) (width 0.25) (layer F.Cu) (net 5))
 (segment (start 64.29739 62.97659) (end 60.26421 62.97659) (width 0.25) (layer F.Cu) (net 5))
 (segment (start 65.0748 63.754) (end 64.29739 62.97659) (width 0.25) (layer F.Cu) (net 5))
 (segment (start 59.6392 63.6016) (end 58.7502 63.6016) (width 0.25) (layer F.Cu) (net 5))
 (segment (start 58.7502 63.6016) (end 58.7502 63.6016) (width 0.25) (layer F.Cu) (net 5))
 (via (at 58.7502 63.6016) (size 0.8) (drill 0.4) (layers F.Cu B.Cu) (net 5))
 (segment (start 58.7502 63.6016) (end 58.0898 64.262) (width 0.25) (layer B.Cu) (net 5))
 (segment (start 58.0898 64.262) (end 58.0898 64.6176) (width 0.25) (layer B.Cu) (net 5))
 (segment (start 58.0898 64.6176) (end 58.928 65.4558) (width 0.25) (layer B.Cu) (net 5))
 (segment (start 60.128002 65.4558) (end 61.737801 67.065599) (width 0.25) (layer B.Cu) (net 5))
 (segment (start 58.928 65.4558) (end 60.128002 65.4558) (width 0.25) (layer B.Cu) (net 5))
 (segment (start 61.737801 67.065599) (end 61.7474 67.075198) (width 0.25) (layer B.Cu) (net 5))
 (via (at 61.737801 67.065599) (size 0.8) (drill 0.4) (layers F.Cu B.Cu) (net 5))
 (segment (start 61.737801 68.310801) (end 61.88 68.453) (width 0.25) (layer F.Cu) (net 5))
 (segment (start 61.737801 67.065599) (end 61.737801 68.310801) (width 0.25) (layer F.Cu) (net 5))
 (segment (start 63.097 71.6915) (end 63.097 71.0785) (width 0.25) (layer B.Cu) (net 4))
 (segment (start 63.097 71.0785) (end 63.53175 70.64375) (width 0.25) (layer B.Cu) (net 4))
 (segment (start 63.53175 70.64375) (end 63.627 70.5485) (width 0.25) (layer B.Cu) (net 4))
 (via (at 63.53175 70.64375) (size 0.8) (drill 0.4) (layers F.Cu B.Cu) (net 4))
 (segment (start 63.53175 70.64375) (end 63.65875 70.64375) (width 0.25) (layer F.Cu) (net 4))
 (segment (start 63.88 70.4225) (end 63.88 68.453) (width 0.25) (layer F.Cu) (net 4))
 (segment (start 63.65875 70.64375) (end 63.88 70.4225) (width 0.25) (layer F.Cu) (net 4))
 (segment (start 68.08419 66.12661) (end 69.263 64.9478) (width 0.25) (layer F.Cu) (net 4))
 (segment (start 67.24879 66.12661) (end 68.08419 66.12661) (width 0.25) (layer F.Cu) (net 4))
 (segment (start 67.424601 63.128099) (end 66.696703 62.400201) (width 0.25) (layer F.Cu) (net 4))
 (segment (start 66.696703 62.400201) (end 59.618831 62.400201) (width 0.25) (layer F.Cu) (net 4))
 (segment (start 67.424601 65.950799) (end 67.424601 63.128099) (width 0.25) (layer F.Cu) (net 4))
 (segment (start 67.24879 66.12661) (end 67.424601 65.950799) (width 0.25) (layer F.Cu) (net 4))
 (segment (start 56.254999 65.764033) (end 56.843916 65.175116) (width 0.25) (layer F.Cu) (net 4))
 (segment (start 56.254999 67.550803) (end 56.254999 65.764033) (width 0.25) (layer F.Cu) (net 4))
 (segment (start 55.313601 68.492201) (end 56.254999 67.550803) (width 0.25) (layer F.Cu) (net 4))
 (segment (start 54.065001 68.492201) (end 55.313601 68.492201) (width 0.25) (layer F.Cu) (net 4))
 (segment (start 56.843916 65.175116) (end 56.429991 65.589041) (width 0.25) (layer F.Cu) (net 4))
 (segment (start 59.142433 62.876599) (end 58.198999 62.876599) (width 0.25) (layer F.Cu) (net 4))
 (segment (start 59.618831 62.400201) (end 59.142433 62.876599) (width 0.25) (layer F.Cu) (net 4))
 (segment (start 51.9656 66.3928) (end 54.065001 68.492201) (width 0.25) (layer F.Cu) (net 4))
 (segment (start 51.9656 65.8826) (end 51.9656 66.3928) (width 0.25) (layer F.Cu) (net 4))
 (segment (start 56.843916 64.231682) (end 58.198999 62.876599) (width 0.25) (layer F.Cu) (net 4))
 (segment (start 56.843916 65.175116) (end 56.843916 64.231682) (width 0.25) (layer F.Cu) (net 4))
 (segment (start 62.042442 66.12661) (end 64.17081 66.12661) (width 0.25) (layer F.Cu) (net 4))
 (segment (start 61.76419 65.848358) (end 62.042442 66.12661) (width 0.25) (layer F.Cu) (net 4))
 (segment (start 61.76419 64.47661) (end 61.76419 65.848358) (width 0.25) (layer F.Cu) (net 4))
 (segment (start 62.6392 63.6016) (end 61.76419 64.47661) (width 0.25) (layer F.Cu) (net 4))
 (segment (start 63.88 66.8792) (end 64.63259 66.12661) (width 0.25) (layer F.Cu) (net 4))
 (segment (start 63.88 68.453) (end 63.88 66.8792) (width 0.25) (layer F.Cu) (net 4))
 (segment (start 64.63259 66.12661) (end 67.24879 66.12661) (width 0.25) (layer F.Cu) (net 4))
 (segment (start 64.17081 66.12661) (end 64.63259 66.12661) (width 0.25) (layer F.Cu) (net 4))
 (segment (start 58.8645 71.6915) (end 58.8645 71.374) (width 0.25) (layer B.Cu) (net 3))
 (segment (start 58.8645 71.374) (end 58.166 70.6755) (width 0.25) (layer B.Cu) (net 3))
 (segment (start 58.166 70.6755) (end 58.166 70.6755) (width 0.25) (layer B.Cu) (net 3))
 (via (at 58.166 70.6755) (size 0.8) (drill 0.4) (layers F.Cu B.Cu) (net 3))
 (segment (start 56.88 69.3895) (end 56.88 68.453) (width 0.25) (layer F.Cu) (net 3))
 (segment (start 58.166 70.6755) (end 56.88 69.3895) (width 0.25) (layer F.Cu) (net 3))
 (via (at 68.3514 64.0334) (size 0.8) (drill 0.4) (layers F.Cu B.Cu) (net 3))
 (segment (start 72.202 64.0588) (end 72.263 63.9978) (width 0.25) (layer F.Cu) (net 3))
 (segment (start 56.88 66.7608) (end 56.88 68.453) (width 0.25) (layer F.Cu) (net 3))
 (segment (start 59.0892 64.5516) (end 56.88 66.7608) (width 0.25) (layer F.Cu) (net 3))
 (segment (start 59.6392 64.5516) (end 59.0892 64.5516) (width 0.25) (layer F.Cu) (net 3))
 (segment (start 53.7718 64.8462) (end 53.7464 64.8716) (width 0.25) (layer B.Cu) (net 3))
 (via (at 53.7718 64.8462) (size 0.8) (drill 0.4) (layers F.Cu B.Cu) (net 3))
 (segment (start 54.8792 64.8462) (end 54.9656 64.9326) (width 0.25) (layer F.Cu) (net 3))
 (segment (start 53.7718 64.8462) (end 54.8792 64.8462) (width 0.25) (layer F.Cu) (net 3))
 (segment (start 59.6392 64.5516) (end 60.0354 64.5516) (width 0.25) (layer F.Cu) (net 3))
 (segment (start 67.945 63.627) (end 68.3514 64.0334) (width 0.25) (layer B.Cu) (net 3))
 (segment (start 60.96 63.627) (end 67.945 63.627) (width 0.25) (layer B.Cu) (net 3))
 (segment (start 72.2274 64.0334) (end 72.263 63.9978) (width 0.25) (layer F.Cu) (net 3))
 (segment (start 68.3514 64.0334) (end 72.2274 64.0334) (width 0.25) (layer F.Cu) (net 3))
 (segment (start 60.110201 62.777201) (end 60.96 63.627) (width 0.25) (layer B.Cu) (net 3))
 (segment (start 55.653602 64.8462) (end 57.722601 62.777201) (width 0.25) (layer B.Cu) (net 3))
 (segment (start 53.7718 64.8462) (end 55.653602 64.8462) (width 0.25) (layer B.Cu) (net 3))
 (segment (start 57.722601 62.777201) (end 60.110201 62.777201) (width 0.25) (layer B.Cu) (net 3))
 (segment (start 59.6392 64.5516) (end 60.706 64.4906) (width 0.25) (layer F.Cu) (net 3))
 (segment (start 60.706 64.4906) (end 60.645 64.5516) (width 0.25) (layer F.Cu) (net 3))
 (via (at 60.706 64.4906) (size 0.8) (drill 0.4) (layers F.Cu B.Cu) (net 3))
 (segment (start 60.706 63.881) (end 60.96 63.627) (width 0.25) (layer B.Cu) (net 3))
 (segment (start 60.706 64.4906) (end 60.706 63.881) (width 0.25) (layer B.Cu) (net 3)))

